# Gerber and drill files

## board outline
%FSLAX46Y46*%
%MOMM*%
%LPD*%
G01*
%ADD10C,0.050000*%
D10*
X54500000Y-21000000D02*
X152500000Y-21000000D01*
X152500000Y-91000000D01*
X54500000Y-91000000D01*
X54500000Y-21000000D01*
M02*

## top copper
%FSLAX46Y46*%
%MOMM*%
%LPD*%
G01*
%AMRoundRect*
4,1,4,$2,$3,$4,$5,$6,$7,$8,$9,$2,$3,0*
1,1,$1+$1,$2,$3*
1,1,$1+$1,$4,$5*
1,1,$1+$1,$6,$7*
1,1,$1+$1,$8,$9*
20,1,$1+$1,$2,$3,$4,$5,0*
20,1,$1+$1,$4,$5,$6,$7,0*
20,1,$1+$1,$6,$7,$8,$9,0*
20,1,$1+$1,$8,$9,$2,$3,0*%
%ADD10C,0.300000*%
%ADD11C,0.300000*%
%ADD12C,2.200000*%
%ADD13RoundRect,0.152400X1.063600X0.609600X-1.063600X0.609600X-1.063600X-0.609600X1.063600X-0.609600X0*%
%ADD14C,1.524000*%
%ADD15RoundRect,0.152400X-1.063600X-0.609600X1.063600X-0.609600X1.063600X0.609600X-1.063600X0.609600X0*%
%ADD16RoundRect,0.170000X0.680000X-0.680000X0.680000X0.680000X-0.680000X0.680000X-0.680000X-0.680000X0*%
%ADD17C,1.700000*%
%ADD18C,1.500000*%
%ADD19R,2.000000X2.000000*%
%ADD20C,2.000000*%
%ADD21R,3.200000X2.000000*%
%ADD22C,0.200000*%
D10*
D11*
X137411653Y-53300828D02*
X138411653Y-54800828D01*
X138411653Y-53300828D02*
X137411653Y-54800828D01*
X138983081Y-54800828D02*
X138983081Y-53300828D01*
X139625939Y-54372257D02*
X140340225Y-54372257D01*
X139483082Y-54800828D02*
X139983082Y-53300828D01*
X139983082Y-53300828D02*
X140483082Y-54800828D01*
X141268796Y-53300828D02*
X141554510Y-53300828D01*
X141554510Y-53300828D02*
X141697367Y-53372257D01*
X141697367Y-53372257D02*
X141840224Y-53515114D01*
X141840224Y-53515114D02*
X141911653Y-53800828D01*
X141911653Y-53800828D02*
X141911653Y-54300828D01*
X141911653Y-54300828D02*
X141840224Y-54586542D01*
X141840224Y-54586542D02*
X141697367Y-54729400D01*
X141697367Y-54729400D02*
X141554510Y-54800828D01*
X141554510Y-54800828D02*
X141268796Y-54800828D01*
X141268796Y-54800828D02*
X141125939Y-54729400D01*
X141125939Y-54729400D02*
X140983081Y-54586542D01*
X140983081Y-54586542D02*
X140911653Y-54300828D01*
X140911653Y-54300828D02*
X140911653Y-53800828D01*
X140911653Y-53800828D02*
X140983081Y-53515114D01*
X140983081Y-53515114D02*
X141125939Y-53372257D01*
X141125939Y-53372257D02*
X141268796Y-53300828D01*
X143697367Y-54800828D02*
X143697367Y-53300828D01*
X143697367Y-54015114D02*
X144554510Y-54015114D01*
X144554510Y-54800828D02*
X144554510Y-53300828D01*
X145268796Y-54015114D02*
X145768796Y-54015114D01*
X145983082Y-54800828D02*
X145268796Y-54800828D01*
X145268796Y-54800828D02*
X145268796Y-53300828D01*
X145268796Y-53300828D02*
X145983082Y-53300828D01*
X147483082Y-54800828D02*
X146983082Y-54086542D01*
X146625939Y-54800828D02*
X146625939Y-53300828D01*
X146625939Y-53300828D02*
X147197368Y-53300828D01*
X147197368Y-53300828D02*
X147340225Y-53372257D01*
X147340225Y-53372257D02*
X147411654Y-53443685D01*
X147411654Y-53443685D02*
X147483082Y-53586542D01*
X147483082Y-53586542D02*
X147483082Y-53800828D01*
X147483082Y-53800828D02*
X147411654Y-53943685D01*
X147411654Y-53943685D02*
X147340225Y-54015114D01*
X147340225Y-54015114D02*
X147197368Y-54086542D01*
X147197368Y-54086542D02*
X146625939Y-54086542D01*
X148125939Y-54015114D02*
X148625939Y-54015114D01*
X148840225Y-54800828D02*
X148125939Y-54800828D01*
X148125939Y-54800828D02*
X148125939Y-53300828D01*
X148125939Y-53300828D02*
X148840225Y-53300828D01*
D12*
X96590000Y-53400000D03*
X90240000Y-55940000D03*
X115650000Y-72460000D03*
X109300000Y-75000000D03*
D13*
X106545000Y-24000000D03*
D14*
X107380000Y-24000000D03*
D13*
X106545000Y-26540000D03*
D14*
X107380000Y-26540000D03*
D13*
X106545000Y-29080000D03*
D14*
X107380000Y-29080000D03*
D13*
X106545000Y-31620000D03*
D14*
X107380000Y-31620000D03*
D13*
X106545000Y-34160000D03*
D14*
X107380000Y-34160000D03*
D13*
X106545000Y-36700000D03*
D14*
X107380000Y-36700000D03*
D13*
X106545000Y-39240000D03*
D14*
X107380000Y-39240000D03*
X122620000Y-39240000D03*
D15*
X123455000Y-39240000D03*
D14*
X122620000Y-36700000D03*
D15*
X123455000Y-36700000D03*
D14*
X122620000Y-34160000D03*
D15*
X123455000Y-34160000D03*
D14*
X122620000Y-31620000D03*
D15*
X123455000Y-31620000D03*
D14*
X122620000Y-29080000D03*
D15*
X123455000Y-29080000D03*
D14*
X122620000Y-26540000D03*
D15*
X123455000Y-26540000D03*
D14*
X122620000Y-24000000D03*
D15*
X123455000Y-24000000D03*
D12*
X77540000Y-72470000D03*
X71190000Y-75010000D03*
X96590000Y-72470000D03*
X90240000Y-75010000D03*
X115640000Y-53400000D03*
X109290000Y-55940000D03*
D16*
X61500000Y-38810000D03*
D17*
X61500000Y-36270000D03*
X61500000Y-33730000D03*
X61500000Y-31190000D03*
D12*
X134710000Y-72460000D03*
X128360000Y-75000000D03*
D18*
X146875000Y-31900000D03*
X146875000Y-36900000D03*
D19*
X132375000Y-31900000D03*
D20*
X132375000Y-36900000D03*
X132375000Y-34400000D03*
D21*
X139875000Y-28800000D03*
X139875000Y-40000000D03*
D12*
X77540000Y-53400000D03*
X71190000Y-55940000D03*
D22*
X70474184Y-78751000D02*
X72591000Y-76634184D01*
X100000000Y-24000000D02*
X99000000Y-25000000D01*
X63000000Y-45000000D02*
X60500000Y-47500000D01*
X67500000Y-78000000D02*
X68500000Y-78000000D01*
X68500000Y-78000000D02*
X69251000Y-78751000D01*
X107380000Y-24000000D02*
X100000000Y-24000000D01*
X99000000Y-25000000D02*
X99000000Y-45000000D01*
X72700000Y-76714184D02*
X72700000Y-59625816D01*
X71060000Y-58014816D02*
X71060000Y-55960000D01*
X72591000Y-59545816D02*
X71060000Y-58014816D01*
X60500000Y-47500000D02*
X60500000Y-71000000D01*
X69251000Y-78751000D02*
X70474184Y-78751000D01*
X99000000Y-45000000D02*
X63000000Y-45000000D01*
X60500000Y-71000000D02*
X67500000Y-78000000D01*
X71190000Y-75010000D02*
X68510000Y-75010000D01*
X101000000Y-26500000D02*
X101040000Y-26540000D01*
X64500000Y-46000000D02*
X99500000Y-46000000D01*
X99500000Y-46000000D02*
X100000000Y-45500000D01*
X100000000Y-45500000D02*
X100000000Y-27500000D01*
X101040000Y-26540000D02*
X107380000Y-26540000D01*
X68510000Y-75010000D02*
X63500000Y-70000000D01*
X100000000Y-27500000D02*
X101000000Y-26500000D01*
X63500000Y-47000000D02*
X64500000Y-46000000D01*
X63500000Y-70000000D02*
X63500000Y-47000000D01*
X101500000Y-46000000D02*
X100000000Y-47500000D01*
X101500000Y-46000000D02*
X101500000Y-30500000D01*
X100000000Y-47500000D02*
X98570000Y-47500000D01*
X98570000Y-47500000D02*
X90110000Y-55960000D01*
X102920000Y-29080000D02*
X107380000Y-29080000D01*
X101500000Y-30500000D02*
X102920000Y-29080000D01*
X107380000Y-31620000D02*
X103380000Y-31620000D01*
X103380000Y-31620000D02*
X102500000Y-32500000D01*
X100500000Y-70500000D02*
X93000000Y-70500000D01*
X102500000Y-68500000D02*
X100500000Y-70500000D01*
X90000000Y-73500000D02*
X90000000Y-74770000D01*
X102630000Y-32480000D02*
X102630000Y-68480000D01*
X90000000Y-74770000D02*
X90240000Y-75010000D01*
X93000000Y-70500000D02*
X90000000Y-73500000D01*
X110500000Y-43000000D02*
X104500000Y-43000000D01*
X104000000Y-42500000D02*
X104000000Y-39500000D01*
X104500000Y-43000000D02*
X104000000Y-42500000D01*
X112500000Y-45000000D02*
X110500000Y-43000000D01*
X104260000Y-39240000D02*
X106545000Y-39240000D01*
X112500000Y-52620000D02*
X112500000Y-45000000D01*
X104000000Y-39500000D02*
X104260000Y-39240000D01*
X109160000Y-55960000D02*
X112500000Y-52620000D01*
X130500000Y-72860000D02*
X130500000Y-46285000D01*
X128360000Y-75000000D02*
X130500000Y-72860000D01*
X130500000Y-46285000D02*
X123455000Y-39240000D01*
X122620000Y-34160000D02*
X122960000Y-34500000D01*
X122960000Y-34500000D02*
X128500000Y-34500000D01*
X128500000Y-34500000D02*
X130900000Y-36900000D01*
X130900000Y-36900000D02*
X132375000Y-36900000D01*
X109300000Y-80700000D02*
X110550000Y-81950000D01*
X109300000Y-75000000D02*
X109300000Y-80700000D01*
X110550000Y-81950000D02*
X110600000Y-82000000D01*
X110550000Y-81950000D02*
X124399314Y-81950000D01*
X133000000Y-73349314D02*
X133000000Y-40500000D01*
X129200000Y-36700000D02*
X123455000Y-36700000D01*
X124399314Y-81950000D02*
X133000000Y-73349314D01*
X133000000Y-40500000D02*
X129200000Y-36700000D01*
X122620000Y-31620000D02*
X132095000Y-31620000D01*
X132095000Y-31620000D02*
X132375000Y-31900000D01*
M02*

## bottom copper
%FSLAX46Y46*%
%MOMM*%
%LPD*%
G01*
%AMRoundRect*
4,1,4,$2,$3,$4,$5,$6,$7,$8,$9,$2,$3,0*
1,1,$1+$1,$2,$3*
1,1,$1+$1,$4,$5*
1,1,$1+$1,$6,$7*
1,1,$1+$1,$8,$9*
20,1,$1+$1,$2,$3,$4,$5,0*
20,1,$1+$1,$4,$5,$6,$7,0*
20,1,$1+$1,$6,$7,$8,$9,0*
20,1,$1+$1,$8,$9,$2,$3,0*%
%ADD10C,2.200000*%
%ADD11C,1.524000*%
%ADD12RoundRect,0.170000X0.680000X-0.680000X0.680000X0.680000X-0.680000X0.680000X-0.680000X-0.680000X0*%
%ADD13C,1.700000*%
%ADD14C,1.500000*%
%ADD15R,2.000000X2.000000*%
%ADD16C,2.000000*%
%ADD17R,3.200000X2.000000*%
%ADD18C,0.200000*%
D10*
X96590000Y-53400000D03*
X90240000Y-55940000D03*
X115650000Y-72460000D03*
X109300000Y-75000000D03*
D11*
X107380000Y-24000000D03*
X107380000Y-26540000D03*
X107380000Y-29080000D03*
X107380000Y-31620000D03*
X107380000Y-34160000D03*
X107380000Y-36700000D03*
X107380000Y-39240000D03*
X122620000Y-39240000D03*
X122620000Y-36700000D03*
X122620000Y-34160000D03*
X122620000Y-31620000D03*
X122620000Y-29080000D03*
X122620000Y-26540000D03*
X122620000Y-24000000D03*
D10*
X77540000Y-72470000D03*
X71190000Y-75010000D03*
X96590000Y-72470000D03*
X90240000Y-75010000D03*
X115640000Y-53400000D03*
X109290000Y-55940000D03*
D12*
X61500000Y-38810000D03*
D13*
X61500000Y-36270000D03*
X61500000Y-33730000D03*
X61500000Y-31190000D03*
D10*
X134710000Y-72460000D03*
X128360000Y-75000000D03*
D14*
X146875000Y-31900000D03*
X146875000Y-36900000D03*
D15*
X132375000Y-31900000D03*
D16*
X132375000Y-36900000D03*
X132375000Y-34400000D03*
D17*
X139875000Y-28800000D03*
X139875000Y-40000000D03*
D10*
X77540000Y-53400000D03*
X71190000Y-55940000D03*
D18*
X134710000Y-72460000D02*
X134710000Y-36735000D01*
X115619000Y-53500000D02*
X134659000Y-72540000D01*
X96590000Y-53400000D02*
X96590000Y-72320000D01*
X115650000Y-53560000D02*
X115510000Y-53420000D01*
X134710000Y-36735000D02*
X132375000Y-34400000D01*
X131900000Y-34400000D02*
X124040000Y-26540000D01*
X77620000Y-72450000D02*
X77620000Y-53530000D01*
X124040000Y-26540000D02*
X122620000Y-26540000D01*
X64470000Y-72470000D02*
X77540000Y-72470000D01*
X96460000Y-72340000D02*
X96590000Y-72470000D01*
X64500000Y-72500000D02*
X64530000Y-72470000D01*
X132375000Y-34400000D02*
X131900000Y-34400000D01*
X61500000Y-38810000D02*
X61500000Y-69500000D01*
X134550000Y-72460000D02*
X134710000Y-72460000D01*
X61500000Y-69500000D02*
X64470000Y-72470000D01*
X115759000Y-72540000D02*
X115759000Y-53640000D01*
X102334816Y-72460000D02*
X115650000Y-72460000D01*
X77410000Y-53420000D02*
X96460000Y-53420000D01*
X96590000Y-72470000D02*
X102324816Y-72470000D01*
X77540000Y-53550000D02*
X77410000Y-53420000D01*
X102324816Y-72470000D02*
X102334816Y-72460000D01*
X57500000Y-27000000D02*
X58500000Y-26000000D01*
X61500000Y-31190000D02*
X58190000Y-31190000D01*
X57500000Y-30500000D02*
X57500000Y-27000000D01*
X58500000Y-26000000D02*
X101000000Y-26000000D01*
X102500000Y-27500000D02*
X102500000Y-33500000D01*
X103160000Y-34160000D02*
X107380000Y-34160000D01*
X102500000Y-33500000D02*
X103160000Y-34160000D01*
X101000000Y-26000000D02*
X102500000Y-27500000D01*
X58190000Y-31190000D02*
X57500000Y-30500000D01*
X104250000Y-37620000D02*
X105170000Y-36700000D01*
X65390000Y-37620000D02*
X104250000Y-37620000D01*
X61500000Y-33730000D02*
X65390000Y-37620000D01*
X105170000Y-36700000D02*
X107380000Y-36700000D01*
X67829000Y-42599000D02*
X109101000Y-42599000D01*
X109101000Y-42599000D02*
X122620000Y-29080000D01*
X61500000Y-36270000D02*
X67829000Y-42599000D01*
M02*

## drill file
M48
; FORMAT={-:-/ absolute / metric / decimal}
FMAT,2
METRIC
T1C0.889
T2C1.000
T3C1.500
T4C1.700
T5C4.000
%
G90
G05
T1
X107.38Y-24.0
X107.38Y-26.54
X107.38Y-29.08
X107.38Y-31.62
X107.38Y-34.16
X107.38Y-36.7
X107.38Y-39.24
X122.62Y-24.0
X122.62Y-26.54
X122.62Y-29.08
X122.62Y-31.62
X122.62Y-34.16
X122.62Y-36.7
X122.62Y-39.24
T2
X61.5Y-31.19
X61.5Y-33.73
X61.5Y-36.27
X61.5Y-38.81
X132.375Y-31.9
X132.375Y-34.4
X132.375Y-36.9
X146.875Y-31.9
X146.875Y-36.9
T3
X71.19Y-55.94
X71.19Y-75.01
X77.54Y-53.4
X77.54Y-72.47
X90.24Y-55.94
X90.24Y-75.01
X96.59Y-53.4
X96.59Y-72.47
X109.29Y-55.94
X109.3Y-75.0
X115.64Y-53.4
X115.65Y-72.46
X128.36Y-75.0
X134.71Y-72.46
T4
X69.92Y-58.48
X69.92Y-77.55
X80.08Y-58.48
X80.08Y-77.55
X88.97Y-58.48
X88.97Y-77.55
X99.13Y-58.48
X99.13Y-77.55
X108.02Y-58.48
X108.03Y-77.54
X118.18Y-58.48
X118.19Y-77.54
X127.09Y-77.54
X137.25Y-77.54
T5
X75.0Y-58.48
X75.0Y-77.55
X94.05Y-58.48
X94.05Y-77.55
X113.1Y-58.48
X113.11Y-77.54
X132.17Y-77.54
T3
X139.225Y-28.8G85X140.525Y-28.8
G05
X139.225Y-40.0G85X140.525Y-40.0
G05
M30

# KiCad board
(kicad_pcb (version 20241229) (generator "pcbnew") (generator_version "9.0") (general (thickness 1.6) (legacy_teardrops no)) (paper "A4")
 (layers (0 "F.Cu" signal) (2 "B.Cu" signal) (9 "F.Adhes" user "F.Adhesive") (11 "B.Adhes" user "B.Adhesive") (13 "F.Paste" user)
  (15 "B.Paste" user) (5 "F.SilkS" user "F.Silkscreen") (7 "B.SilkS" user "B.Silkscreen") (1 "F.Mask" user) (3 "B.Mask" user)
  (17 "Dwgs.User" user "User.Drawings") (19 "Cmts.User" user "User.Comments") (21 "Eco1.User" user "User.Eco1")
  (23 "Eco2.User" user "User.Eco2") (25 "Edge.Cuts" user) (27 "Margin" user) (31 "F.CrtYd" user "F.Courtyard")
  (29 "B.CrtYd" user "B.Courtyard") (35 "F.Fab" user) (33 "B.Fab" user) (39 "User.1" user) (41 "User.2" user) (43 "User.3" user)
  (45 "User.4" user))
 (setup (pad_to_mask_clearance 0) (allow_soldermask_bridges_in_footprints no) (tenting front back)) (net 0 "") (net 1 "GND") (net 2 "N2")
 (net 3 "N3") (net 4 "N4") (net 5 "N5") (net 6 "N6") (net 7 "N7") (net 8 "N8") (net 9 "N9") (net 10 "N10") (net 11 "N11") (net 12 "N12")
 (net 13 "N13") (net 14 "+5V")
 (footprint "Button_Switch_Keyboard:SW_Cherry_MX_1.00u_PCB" (layer "F.Cu") (at 96.59 53.4)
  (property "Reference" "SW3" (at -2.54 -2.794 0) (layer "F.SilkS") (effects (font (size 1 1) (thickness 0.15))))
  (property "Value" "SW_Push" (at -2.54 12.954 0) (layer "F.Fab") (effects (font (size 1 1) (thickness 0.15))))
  (pad "" np_thru_hole circle (at -7.62 5.08) (size 1.7 1.7) (drill 1.7) (layers "*.Cu" "*.Mask"))
  (pad "" np_thru_hole circle (at -2.54 5.08) (size 4 4) (drill 4) (layers "*.Cu" "*.Mask"))
  (pad "" np_thru_hole circle (at 2.54 5.08) (size 1.7 1.7) (drill 1.7) (layers "*.Cu" "*.Mask"))
  (pad "1" thru_hole circle (at 0 0) (size 2.2 2.2) (drill 1.5) (layers "*.Cu" "*.Mask") (remove_unused_layers no) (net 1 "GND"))
  (pad "2" thru_hole circle (at -6.35 2.54) (size 2.2 2.2) (drill 1.5) (layers "*.Cu" "*.Mask") (remove_unused_layers no) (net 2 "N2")))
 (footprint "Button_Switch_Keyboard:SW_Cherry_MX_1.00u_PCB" (layer "F.Cu") (at 115.65 72.46)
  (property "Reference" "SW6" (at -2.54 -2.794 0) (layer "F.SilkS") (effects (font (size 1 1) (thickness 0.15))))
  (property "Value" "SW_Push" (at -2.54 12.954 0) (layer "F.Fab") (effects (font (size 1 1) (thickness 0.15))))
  (pad "" np_thru_hole circle (at -7.62 5.08) (size 1.7 1.7) (drill 1.7) (layers "*.Cu" "*.Mask"))
  (pad "" np_thru_hole circle (at -2.54 5.08) (size 4 4) (drill 4) (layers "*.Cu" "*.Mask"))
  (pad "" np_thru_hole circle (at 2.54 5.08) (size 1.7 1.7) (drill 1.7) (layers "*.Cu" "*.Mask"))
  (pad "1" thru_hole circle (at 0 0) (size 2.2 2.2) (drill 1.5) (layers "*.Cu" "*.Mask") (remove_unused_layers no) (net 1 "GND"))
  (pad "2" thru_hole circle (at -6.35 2.54) (size 2.2 2.2) (drill 1.5) (layers "*.Cu" "*.Mask") (remove_unused_layers no) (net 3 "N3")))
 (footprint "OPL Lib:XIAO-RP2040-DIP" (layer "F.Cu") (at 115 31.62)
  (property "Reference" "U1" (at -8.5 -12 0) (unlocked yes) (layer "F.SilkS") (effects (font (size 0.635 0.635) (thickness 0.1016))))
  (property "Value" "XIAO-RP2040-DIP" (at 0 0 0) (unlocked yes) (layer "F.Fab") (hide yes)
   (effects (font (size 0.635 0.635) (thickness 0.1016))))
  (pad "1" smd roundrect (at -8.455 -7.62 180) (size 2.432 1.524) (layers "F.Cu" "F.Mask") (roundrect_rratio 0.1) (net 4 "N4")
   (thermal_bridge_angle 45))
  (pad "1" thru_hole circle (at -7.62 -7.62 180) (size 1.524 1.524) (drill 0.889) (layers "*.Cu" "*.Mask") (remove_unused_layers no)
   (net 4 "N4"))
  (pad "2" smd roundrect (at -8.455 -5.08 180) (size 2.432 1.524) (layers "F.Cu" "F.Mask") (roundrect_rratio 0.1) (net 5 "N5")
   (thermal_bridge_angle 45))
  (pad "2" thru_hole circle (at -7.62 -5.08 180) (size 1.524 1.524) (drill 0.889) (layers "*.Cu" "*.Mask") (remove_unused_layers no)
   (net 5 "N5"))
  (pad "3" smd roundrect (at -8.455 -2.54 180) (size 2.432 1.524) (layers "F.Cu" "F.Mask") (roundrect_rratio 0.1) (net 2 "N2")
   (thermal_bridge_angle 45))
  (pad "3" thru_hole circle (at -7.62 -2.54 180) (size 1.524 1.524) (drill 0.889) (layers "*.Cu" "*.Mask") (remove_unused_layers no)
   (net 2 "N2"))
  (pad "4" smd roundrect (at -8.455 0 180) (size 2.432 1.524) (layers "F.Cu" "F.Mask") (roundrect_rratio 0.1) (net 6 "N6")
   (thermal_bridge_angle 45))
  (pad "4" thru_hole circle (at -7.62 0 180) (size 1.524 1.524) (drill 0.889) (layers "*.Cu" "*.Mask") (remove_unused_layers no)
   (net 6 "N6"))
  (pad "5" smd roundrect (at -8.455 2.54 180) (size 2.432 1.524) (layers "F.Cu" "F.Mask") (roundrect_rratio 0.1) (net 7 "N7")
   (thermal_bridge_angle 45))
  (pad "5" thru_hole circle (at -7.62 2.54 180) (size 1.524 1.524) (drill 0.889) (layers "*.Cu" "*.Mask") (remove_unused_layers no)
   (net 7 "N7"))
  (pad "6" smd roundrect (at -8.455 5.08 180) (size 2.432 1.524) (layers "F.Cu" "F.Mask") (roundrect_rratio 0.1) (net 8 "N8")
   (thermal_bridge_angle 45))
  (pad "6" thru_hole circle (at -7.62 5.08 180) (size 1.524 1.524) (drill 0.889) (layers "*.Cu" "*.Mask") (remove_unused_layers no)
   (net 8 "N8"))
  (pad "7" smd roundrect (at -8.455 7.62 180) (size 2.432 1.524) (layers "F.Cu" "F.Mask") (roundrect_rratio 0.1) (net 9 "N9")
   (thermal_bridge_angle 45))
  (pad "7" thru_hole circle (at -7.62 7.62 180) (size 1.524 1.524) (drill 0.889) (layers "*.Cu" "*.Mask") (remove_unused_layers no)
   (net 9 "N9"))
  (pad "8" thru_hole circle (at 7.62 7.62) (size 1.524 1.524) (drill 0.889) (layers "*.Cu" "*.Mask") (remove_unused_layers no)
   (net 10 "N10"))
  (pad "8" smd roundrect (at 8.455 7.62) (size 2.432 1.524) (layers "F.Cu" "F.Mask") (roundrect_rratio 0.1) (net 10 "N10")
   (thermal_bridge_angle 45))
  (pad "9" thru_hole circle (at 7.62 5.08) (size 1.524 1.524) (drill 0.889) (layers "*.Cu" "*.Mask") (remove_unused_layers no) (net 3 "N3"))
  (pad "9" smd roundrect (at 8.455 5.08) (size 2.432 1.524) (layers "F.Cu" "F.Mask") (roundrect_rratio 0.1) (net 3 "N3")
   (thermal_bridge_angle 45))
  (pad "10" thru_hole circle (at 7.62 2.54) (size 1.524 1.524) (drill 0.889) (layers "*.Cu" "*.Mask") (remove_unused_layers no)
   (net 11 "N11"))
  (pad "10" smd roundrect (at 8.455 2.54) (size 2.432 1.524) (layers "F.Cu" "F.Mask") (roundrect_rratio 0.1) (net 11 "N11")
   (thermal_bridge_angle 45))
  (pad "11" thru_hole circle (at 7.62 0) (size 1.524 1.524) (drill 0.889) (layers "*.Cu" "*.Mask") (remove_unused_layers no) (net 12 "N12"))
  (pad "11" smd roundrect (at 8.455 0) (size 2.432 1.524) (layers "F.Cu" "F.Mask") (roundrect_rratio 0.1) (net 12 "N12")
   (thermal_bridge_angle 45))
  (pad "12" thru_hole circle (at 7.62 -2.54) (size 1.524 1.524) (drill 0.889) (layers "*.Cu" "*.Mask") (remove_unused_layers no)
   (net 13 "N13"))
  (pad "12" smd roundrect (at 8.455 -2.54) (size 2.432 1.524) (layers "F.Cu" "F.Mask") (roundrect_rratio 0.1) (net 13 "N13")
   (thermal_bridge_angle 45))
  (pad "13" thru_hole circle (at 7.62 -5.08) (size 1.524 1.524) (drill 0.889) (layers "*.Cu" "*.Mask") (remove_unused_layers no)
   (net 1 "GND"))
  (pad "13" smd roundrect (at 8.455 -5.08) (size 2.432 1.524) (layers "F.Cu" "F.Mask") (roundrect_rratio 0.1) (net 1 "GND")
   (thermal_bridge_angle 45))
  (pad "14" thru_hole circle (at 7.62 -7.62) (size 1.524 1.524) (drill 0.889) (layers "*.Cu" "*.Mask") (remove_unused_layers no)
   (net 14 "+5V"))
  (pad "14" smd roundrect (at 8.455 -7.62) (size 2.432 1.524) (layers "F.Cu" "F.Mask") (roundrect_rratio 0.1) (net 14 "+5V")
   (thermal_bridge_angle 45)))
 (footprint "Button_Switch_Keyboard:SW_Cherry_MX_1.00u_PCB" (layer "F.Cu") (at 77.54 72.47)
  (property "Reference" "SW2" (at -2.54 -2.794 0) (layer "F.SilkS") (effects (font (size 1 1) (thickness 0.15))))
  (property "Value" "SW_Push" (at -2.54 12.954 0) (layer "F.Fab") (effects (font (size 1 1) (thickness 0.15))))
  (pad "" np_thru_hole circle (at -7.62 5.08) (size 1.7 1.7) (drill 1.7) (layers "*.Cu" "*.Mask"))
  (pad "" np_thru_hole circle (at -2.54 5.08) (size 4 4) (drill 4) (layers "*.Cu" "*.Mask"))
  (pad "" np_thru_hole circle (at 2.54 5.08) (size 1.7 1.7) (drill 1.7) (layers "*.Cu" "*.Mask"))
  (pad "1" thru_hole circle (at 0 0) (size 2.2 2.2) (drill 1.5) (layers "*.Cu" "*.Mask") (remove_unused_layers no) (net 1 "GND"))
  (pad "2" thru_hole circle (at -6.35 2.54) (size 2.2 2.2) (drill 1.5) (layers "*.Cu" "*.Mask") (remove_unused_layers no) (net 5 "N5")))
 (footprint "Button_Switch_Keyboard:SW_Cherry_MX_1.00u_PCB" (layer "F.Cu") (at 96.59 72.47)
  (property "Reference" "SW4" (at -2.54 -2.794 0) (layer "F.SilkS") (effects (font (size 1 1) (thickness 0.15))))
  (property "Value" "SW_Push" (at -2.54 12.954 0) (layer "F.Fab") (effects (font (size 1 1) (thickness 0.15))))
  (pad "" np_thru_hole circle (at -7.62 5.08) (size 1.7 1.7) (drill 1.7) (layers "*.Cu" "*.Mask"))
  (pad "" np_thru_hole circle (at -2.54 5.08) (size 4 4) (drill 4) (layers "*.Cu" "*.Mask"))
  (pad "" np_thru_hole circle (at 2.54 5.08) (size 1.7 1.7) (drill 1.7) (layers "*.Cu" "*.Mask"))
  (pad "1" thru_hole circle (at 0 0) (size 2.2 2.2) (drill 1.5) (layers "*.Cu" "*.Mask") (remove_unused_layers no) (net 1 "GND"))
  (pad "2" thru_hole circle (at -6.35 2.54) (size 2.2 2.2) (drill 1.5) (layers "*.Cu" "*.Mask") (remove_unused_layers no) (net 6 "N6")))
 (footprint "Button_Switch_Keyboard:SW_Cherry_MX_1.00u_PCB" (layer "F.Cu") (at 115.64 53.4)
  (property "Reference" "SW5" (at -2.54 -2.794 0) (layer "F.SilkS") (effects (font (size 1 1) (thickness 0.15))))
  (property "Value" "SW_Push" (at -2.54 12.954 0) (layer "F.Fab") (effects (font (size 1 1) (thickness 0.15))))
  (pad "" np_thru_hole circle (at -7.62 5.08) (size 1.7 1.7) (drill 1.7) (layers "*.Cu" "*.Mask"))
  (pad "" np_thru_hole circle (at -2.54 5.08) (size 4 4) (drill 4) (layers "*.Cu" "*.Mask"))
  (pad "" np_thru_hole circle (at 2.54 5.08) (size 1.7 1.7) (drill 1.7) (layers "*.Cu" "*.Mask"))
  (pad "1" thru_hole circle (at 0 0) (size 2.2 2.2) (drill 1.5) (layers "*.Cu" "*.Mask") (remove_unused_layers no) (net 1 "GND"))
  (pad "2" thru_hole circle (at -6.35 2.54) (size 2.2 2.2) (drill 1.5) (layers "*.Cu" "*.Mask") (remove_unused_layers no) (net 9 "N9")))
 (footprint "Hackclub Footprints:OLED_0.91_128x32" (layer "F.Cu") (at 61.5 38.81 90)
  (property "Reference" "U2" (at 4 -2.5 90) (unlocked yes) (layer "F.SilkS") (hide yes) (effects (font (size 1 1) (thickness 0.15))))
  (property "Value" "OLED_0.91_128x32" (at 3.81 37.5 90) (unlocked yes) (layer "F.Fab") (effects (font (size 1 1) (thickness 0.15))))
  (pad "1" thru_hole roundrect (at 0 0 90) (size 1.7 1.7) (drill 1) (layers "*.Cu" "*.Mask") (remove_unused_layers no)
   (roundrect_rratio 0.1) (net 1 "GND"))
  (pad "2" thru_hole circle (at 2.54 0 90) (size 1.7 1.7) (drill 1) (layers "*.Cu" "*.Mask") (remove_unused_layers no) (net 13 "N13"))
  (pad "3" thru_hole circle (at 5.08 0 90) (size 1.7 1.7) (drill 1) (layers "*.Cu" "*.Mask") (remove_unused_layers no) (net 8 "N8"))
  (pad "4" thru_hole circle (at 7.62 0 90) (size 1.7 1.7) (drill 1) (layers "*.Cu" "*.Mask") (remove_unused_layers no) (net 7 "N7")))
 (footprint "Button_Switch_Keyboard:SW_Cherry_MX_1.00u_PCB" (layer "F.Cu") (at 134.71 72.46)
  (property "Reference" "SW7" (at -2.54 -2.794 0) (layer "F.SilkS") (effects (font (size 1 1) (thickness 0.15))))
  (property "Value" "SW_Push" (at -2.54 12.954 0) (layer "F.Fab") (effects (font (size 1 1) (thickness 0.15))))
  (pad "" np_thru_hole circle (at -7.62 5.08) (size 1.7 1.7) (drill 1.7) (layers "*.Cu" "*.Mask"))
  (pad "" np_thru_hole circle (at -2.54 5.08) (size 4 4) (drill 4) (layers "*.Cu" "*.Mask"))
  (pad "" np_thru_hole circle (at 2.54 5.08) (size 1.7 1.7) (drill 1.7) (layers "*.Cu" "*.Mask"))
  (pad "1" thru_hole circle (at 0 0) (size 2.2 2.2) (drill 1.5) (layers "*.Cu" "*.Mask") (remove_unused_layers no) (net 1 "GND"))
  (pad "2" thru_hole circle (at -6.35 2.54) (size 2.2 2.2) (drill 1.5) (layers "*.Cu" "*.Mask") (remove_unused_layers no) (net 10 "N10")))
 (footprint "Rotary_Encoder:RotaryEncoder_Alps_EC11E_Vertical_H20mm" (layer "F.Cu") (at 132.375 31.9)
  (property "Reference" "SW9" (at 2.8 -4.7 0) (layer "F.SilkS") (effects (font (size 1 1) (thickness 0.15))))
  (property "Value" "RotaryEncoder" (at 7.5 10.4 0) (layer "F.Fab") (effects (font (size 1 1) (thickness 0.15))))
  (pad "" thru_hole circle (at 14.5 0) (size 1.5 1.5) (drill 1) (layers "*.Cu" "*.Mask") (remove_unused_layers no))
  (pad "" thru_hole circle (at 14.5 5) (size 1.5 1.5) (drill 1) (layers "*.Cu" "*.Mask") (remove_unused_layers no))
  (pad "A" thru_hole rect (at 0 0) (size 2 2) (drill 1) (layers "*.Cu" "*.Mask") (remove_unused_layers no) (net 12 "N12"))
  (pad "B" thru_hole circle (at 0 5) (size 2 2) (drill 1) (layers "*.Cu" "*.Mask") (remove_unused_layers no) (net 11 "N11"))
  (pad "C" thru_hole circle (at 0 2.5) (size 2 2) (drill 1) (layers "*.Cu" "*.Mask") (remove_unused_layers no) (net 1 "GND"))
  (pad "MP" thru_hole rect (at 7.5 -3.1) (size 3.2 2) (drill oval 2.8 1.5) (layers "*.Cu" "*.Mask") (remove_unused_layers no))
  (pad "MP" thru_hole rect (at 7.5 8.1) (size 3.2 2) (drill oval 2.8 1.5) (layers "*.Cu" "*.Mask") (remove_unused_layers no)))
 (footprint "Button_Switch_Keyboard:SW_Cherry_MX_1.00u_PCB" (layer "F.Cu") (at 77.54 53.4)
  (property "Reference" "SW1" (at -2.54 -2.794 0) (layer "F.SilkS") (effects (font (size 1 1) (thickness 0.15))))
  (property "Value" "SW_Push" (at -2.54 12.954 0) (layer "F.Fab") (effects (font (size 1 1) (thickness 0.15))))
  (pad "" np_thru_hole circle (at -7.62 5.08) (size 1.7 1.7) (drill 1.7) (layers "*.Cu" "*.Mask"))
  (pad "" np_thru_hole circle (at -2.54 5.08) (size 4 4) (drill 4) (layers "*.Cu" "*.Mask"))
  (pad "" np_thru_hole circle (at 2.54 5.08) (size 1.7 1.7) (drill 1.7) (layers "*.Cu" "*.Mask"))
  (pad "1" thru_hole circle (at 0 0) (size 2.2 2.2) (drill 1.5) (layers "*.Cu" "*.Mask") (remove_unused_layers no) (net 1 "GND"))
  (pad "2" thru_hole circle (at -6.35 2.54) (size 2.2 2.2) (drill 1.5) (layers "*.Cu" "*.Mask") (remove_unused_layers no) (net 4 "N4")))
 (gr_rect (start 54.5 21) (end 152.5 91) (stroke (width 0.05) (type default)) (fill no) (layer "Edge.Cuts"))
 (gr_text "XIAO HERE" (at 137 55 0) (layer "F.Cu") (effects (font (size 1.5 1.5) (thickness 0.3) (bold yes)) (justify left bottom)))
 (segment (start 134.71 72.46) (end 134.71 36.735) (width 0.2) (layer "B.Cu") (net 1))
 (segment (start 115.619 53.5) (end 134.659 72.54) (width 0.2) (layer "B.Cu") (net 1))
 (segment (start 96.59 53.4) (end 96.59 72.32) (width 0.2) (layer "B.Cu") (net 1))
 (segment (start 115.65 53.56) (end 115.51 53.42) (width 0.2) (layer "B.Cu") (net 1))
 (segment (start 134.71 36.735) (end 132.375 34.4) (width 0.2) (layer "B.Cu") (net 1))
 (segment (start 131.9 34.4) (end 124.04 26.54) (width 0.2) (layer "B.Cu") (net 1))
 (segment (start 77.62 72.45) (end 77.62 53.53) (width 0.2) (layer "B.Cu") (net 1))
 (segment (start 124.04 26.54) (end 122.62 26.54) (width 0.2) (layer "B.Cu") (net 1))
 (segment (start 64.47 72.47) (end 77.54 72.47) (width 0.2) (layer "B.Cu") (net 1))
 (segment (start 96.46 72.34) (end 96.59 72.47) (width 0.2) (layer "B.Cu") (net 1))
 (segment (start 64.5 72.5) (end 64.53 72.47) (width 0.2) (layer "B.Cu") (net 1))
 (segment (start 132.375 34.4) (end 131.9 34.4) (width 0.2) (layer "B.Cu") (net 1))
 (segment (start 61.5 38.81) (end 61.5 69.5) (width 0.2) (layer "B.Cu") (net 1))
 (segment (start 134.55 72.46) (end 134.71 72.46) (width 0.2) (layer "B.Cu") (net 1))
 (segment (start 61.5 69.5) (end 64.47 72.47) (width 0.2) (layer "B.Cu") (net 1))
 (segment (start 115.759 72.54) (end 115.759 53.64) (width 0.2) (layer "B.Cu") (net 1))
 (segment (start 102.334816 72.46) (end 115.65 72.46) (width 0.2) (layer "B.Cu") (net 1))
 (segment (start 77.41 53.42) (end 96.46 53.42) (width 0.2) (layer "B.Cu") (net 1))
 (segment (start 96.59 72.47) (end 102.324816 72.47) (width 0.2) (layer "B.Cu") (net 1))
 (segment (start 77.54 53.55) (end 77.41 53.42) (width 0.2) (layer "B.Cu") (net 1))
 (segment (start 102.324816 72.47) (end 102.334816 72.46) (width 0.2) (layer "B.Cu") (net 1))
 (segment (start 70.474184 78.751) (end 72.591 76.634184) (width 0.2) (layer "F.Cu") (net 4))
 (segment (start 100 24) (end 99 25) (width 0.2) (layer "F.Cu") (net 4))
 (segment (start 63 45) (end 60.5 47.5) (width 0.2) (layer "F.Cu") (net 4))
 (segment (start 67.5 78) (end 68.5 78) (width 0.2) (layer "F.Cu") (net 4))
 (segment (start 68.5 78) (end 69.251 78.751) (width 0.2) (layer "F.Cu") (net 4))
 (segment (start 107.38 24) (end 100 24) (width 0.2) (layer "F.Cu") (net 4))
 (segment (start 99 25) (end 99 45) (width 0.2) (layer "F.Cu") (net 4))
 (segment (start 72.7 76.714184) (end 72.7 59.625816) (width 0.2) (layer "F.Cu") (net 4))
 (segment (start 71.06 58.014816) (end 71.06 55.96) (width 0.2) (layer "F.Cu") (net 4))
 (segment (start 72.591 59.545816) (end 71.06 58.014816) (width 0.2) (layer "F.Cu") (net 4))
 (segment (start 60.5 47.5) (end 60.5 71) (width 0.2) (layer "F.Cu") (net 4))
 (segment (start 69.251 78.751) (end 70.474184 78.751) (width 0.2) (layer "F.Cu") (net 4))
 (segment (start 99 45) (end 63 45) (width 0.2) (layer "F.Cu") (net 4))
 (segment (start 60.5 71) (end 67.5 78) (width 0.2) (layer "F.Cu") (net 4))
 (segment (start 71.19 75.01) (end 68.51 75.01) (width 0.2) (layer "F.Cu") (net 5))
 (segment (start 101 26.5) (end 101.04 26.54) (width 0.2) (layer "F.Cu") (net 5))
 (segment (start 64.5 46) (end 99.5 46) (width 0.2) (layer "F.Cu") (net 5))
 (segment (start 99.5 46) (end 100 45.5) (width 0.2) (layer "F.Cu") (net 5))
 (segment (start 100 45.5) (end 100 27.5) (width 0.2) (layer "F.Cu") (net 5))
 (segment (start 101.04 26.54) (end 107.38 26.54) (width 0.2) (layer "F.Cu") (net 5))
 (segment (start 68.51 75.01) (end 63.5 70) (width 0.2) (layer "F.Cu") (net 5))
 (segment (start 100 27.5) (end 101 26.5) (width 0.2) (layer "F.Cu") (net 5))
 (segment (start 63.5 47) (end 64.5 46) (width 0.2) (layer "F.Cu") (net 5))
 (segment (start 63.5 70) (end 63.5 47) (width 0.2) (layer "F.Cu") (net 5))
 (segment (start 101.5 46) (end 100 47.5) (width 0.2) (layer "F.Cu") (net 2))
 (segment (start 101.5 46) (end 101.5 30.5) (width 0.2) (layer "F.Cu") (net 2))
 (segment (start 100 47.5) (end 98.57 47.5) (width 0.2) (layer "F.Cu") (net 2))
 (segment (start 98.57 47.5) (end 90.11 55.96) (width 0.2) (layer "F.Cu") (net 2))
 (segment (start 102.92 29.08) (end 107.38 29.08) (width 0.2) (layer "F.Cu") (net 2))
 (segment (start 101.5 30.5) (end 102.92 29.08) (width 0.2) (layer "F.Cu") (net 2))
 (segment (start 107.38 31.62) (end 103.38 31.62) (width 0.2) (layer "F.Cu") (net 6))
 (segment (start 103.38 31.62) (end 102.5 32.5) (width 0.2) (layer "F.Cu") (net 6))
 (segment (start 100.5 70.5) (end 93 70.5) (width 0.2) (layer "F.Cu") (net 6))
 (segment (start 102.5 68.5) (end 100.5 70.5) (width 0.2) (layer "F.Cu") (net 6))
 (segment (start 90 73.5) (end 90 74.77) (width 0.2) (layer "F.Cu") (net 6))
 (segment (start 102.63 32.48) (end 102.63 68.48) (width 0.2) (layer "F.Cu") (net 6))
 (segment (start 90 74.77) (end 90.24 75.01) (width 0.2) (layer "F.Cu") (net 6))
 (segment (start 93 70.5) (end 90 73.5) (width 0.2) (layer "F.Cu") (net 6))
 (segment (start 57.5 27) (end 58.5 26) (width 0.2) (layer "B.Cu") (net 7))
 (segment (start 61.5 31.19) (end 58.19 31.19) (width 0.2) (layer "B.Cu") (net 7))
 (segment (start 57.5 30.5) (end 57.5 27) (width 0.2) (layer "B.Cu") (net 7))
 (segment (start 58.5 26) (end 101 26) (width 0.2) (layer "B.Cu") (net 7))
 (segment (start 102.5 27.5) (end 102.5 33.5) (width 0.2) (layer "B.Cu") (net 7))
 (segment (start 103.16 34.16) (end 107.38 34.16) (width 0.2) (layer "B.Cu") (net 7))
 (segment (start 102.5 33.5) (end 103.16 34.16) (width 0.2) (layer "B.Cu") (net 7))
 (segment (start 101 26) (end 102.5 27.5) (width 0.2) (layer "B.Cu") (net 7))
 (segment (start 58.19 31.19) (end 57.5 30.5) (width 0.2) (layer "B.Cu") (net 7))
 (segment (start 104.25 37.62) (end 105.17 36.7) (width 0.2) (layer "B.Cu") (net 8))
 (segment (start 65.39 37.62) (end 104.25 37.62) (width 0.2) (layer "B.Cu") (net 8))
 (segment (start 61.5 33.73) (end 65.39 37.62) (width 0.2) (layer "B.Cu") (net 8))
 (segment (start 105.17 36.7) (end 107.38 36.7) (width 0.2) (layer "B.Cu") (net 8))
 (segment (start 110.5 43) (end 104.5 43) (width 0.2) (layer "F.Cu") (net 9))
 (segment (start 104 42.5) (end 104 39.5) (width 0.2) (layer "F.Cu") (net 9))
 (segment (start 104.5 43) (end 104 42.5) (width 0.2) (layer "F.Cu") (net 9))
 (segment (start 112.5 45) (end 110.5 43) (width 0.2) (layer "F.Cu") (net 9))
 (segment (start 104.26 39.24) (end 106.545 39.24) (width 0.2) (layer "F.Cu") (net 9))
 (segment (start 112.5 52.62) (end 112.5 45) (width 0.2) (layer "F.Cu") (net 9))
 (segment (start 104 39.5) (end 104.26 39.24) (width 0.2) (layer "F.Cu") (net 9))
 (segment (start 109.16 55.96) (end 112.5 52.62) (width 0.2) (layer "F.Cu") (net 9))
 (segment (start 130.5 72.86) (end 130.5 46.285) (width 0.2) (layer "F.Cu") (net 10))
 (segment (start 128.36 75) (end 130.5 72.86) (width 0.2) (layer "F.Cu") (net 10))
 (segment (start 130.5 46.285) (end 123.455 39.24) (width 0.2) (layer "F.Cu") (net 10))
 (segment (start 122.62 34.16) (end 122.96 34.5) (width 0.2) (layer "F.Cu") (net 11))
 (segment (start 122.96 34.5) (end 128.5 34.5) (width 0.2) (layer "F.Cu") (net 11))
 (segment (start 128.5 34.5) (end 130.9 36.9) (width 0.2) (layer "F.Cu") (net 11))
 (segment (start 130.9 36.9) (end 132.375 36.9) (width 0.2) (layer "F.Cu") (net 11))
 (segment (start 109.3 80.7) (end 110.55 81.95) (width 0.2) (layer "F.Cu") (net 3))
 (segment (start 109.3 75) (end 109.3 80.7) (width 0.2) (layer "F.Cu") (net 3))
 (segment (start 110.55 81.95) (end 110.6 82) (width 0.2) (layer "F.Cu") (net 3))
 (segment (start 110.55 81.95) (end 124.399314 81.95) (width 0.2) (layer "F.Cu") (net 3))
 (segment (start 133 73.349314) (end 133 40.5) (width 0.2) (layer "F.Cu") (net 3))
 (segment (start 129.2 36.7) (end 123.455 36.7) (width 0.2) (layer "F.Cu") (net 3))
 (segment (start 124.399314 81.95) (end 133 73.349314) (width 0.2) (layer "F.Cu") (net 3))
 (segment (start 133 40.5) (end 129.2 36.7) (width 0.2) (layer "F.Cu") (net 3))
 (segment (start 122.62 31.62) (end 132.095 31.62) (width 0.2) (layer "F.Cu") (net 12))
 (segment (start 132.095 31.62) (end 132.375 31.9) (width 0.2) (layer "F.Cu") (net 12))
 (segment (start 67.829 42.599) (end 109.101 42.599) (width 0.2) (layer "B.Cu") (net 13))
 (segment (start 109.101 42.599) (end 122.62 29.08) (width 0.2) (layer "B.Cu") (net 13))
 (segment (start 61.5 36.27) (end 67.829 42.599) (width 0.2) (layer "B.Cu") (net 13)))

